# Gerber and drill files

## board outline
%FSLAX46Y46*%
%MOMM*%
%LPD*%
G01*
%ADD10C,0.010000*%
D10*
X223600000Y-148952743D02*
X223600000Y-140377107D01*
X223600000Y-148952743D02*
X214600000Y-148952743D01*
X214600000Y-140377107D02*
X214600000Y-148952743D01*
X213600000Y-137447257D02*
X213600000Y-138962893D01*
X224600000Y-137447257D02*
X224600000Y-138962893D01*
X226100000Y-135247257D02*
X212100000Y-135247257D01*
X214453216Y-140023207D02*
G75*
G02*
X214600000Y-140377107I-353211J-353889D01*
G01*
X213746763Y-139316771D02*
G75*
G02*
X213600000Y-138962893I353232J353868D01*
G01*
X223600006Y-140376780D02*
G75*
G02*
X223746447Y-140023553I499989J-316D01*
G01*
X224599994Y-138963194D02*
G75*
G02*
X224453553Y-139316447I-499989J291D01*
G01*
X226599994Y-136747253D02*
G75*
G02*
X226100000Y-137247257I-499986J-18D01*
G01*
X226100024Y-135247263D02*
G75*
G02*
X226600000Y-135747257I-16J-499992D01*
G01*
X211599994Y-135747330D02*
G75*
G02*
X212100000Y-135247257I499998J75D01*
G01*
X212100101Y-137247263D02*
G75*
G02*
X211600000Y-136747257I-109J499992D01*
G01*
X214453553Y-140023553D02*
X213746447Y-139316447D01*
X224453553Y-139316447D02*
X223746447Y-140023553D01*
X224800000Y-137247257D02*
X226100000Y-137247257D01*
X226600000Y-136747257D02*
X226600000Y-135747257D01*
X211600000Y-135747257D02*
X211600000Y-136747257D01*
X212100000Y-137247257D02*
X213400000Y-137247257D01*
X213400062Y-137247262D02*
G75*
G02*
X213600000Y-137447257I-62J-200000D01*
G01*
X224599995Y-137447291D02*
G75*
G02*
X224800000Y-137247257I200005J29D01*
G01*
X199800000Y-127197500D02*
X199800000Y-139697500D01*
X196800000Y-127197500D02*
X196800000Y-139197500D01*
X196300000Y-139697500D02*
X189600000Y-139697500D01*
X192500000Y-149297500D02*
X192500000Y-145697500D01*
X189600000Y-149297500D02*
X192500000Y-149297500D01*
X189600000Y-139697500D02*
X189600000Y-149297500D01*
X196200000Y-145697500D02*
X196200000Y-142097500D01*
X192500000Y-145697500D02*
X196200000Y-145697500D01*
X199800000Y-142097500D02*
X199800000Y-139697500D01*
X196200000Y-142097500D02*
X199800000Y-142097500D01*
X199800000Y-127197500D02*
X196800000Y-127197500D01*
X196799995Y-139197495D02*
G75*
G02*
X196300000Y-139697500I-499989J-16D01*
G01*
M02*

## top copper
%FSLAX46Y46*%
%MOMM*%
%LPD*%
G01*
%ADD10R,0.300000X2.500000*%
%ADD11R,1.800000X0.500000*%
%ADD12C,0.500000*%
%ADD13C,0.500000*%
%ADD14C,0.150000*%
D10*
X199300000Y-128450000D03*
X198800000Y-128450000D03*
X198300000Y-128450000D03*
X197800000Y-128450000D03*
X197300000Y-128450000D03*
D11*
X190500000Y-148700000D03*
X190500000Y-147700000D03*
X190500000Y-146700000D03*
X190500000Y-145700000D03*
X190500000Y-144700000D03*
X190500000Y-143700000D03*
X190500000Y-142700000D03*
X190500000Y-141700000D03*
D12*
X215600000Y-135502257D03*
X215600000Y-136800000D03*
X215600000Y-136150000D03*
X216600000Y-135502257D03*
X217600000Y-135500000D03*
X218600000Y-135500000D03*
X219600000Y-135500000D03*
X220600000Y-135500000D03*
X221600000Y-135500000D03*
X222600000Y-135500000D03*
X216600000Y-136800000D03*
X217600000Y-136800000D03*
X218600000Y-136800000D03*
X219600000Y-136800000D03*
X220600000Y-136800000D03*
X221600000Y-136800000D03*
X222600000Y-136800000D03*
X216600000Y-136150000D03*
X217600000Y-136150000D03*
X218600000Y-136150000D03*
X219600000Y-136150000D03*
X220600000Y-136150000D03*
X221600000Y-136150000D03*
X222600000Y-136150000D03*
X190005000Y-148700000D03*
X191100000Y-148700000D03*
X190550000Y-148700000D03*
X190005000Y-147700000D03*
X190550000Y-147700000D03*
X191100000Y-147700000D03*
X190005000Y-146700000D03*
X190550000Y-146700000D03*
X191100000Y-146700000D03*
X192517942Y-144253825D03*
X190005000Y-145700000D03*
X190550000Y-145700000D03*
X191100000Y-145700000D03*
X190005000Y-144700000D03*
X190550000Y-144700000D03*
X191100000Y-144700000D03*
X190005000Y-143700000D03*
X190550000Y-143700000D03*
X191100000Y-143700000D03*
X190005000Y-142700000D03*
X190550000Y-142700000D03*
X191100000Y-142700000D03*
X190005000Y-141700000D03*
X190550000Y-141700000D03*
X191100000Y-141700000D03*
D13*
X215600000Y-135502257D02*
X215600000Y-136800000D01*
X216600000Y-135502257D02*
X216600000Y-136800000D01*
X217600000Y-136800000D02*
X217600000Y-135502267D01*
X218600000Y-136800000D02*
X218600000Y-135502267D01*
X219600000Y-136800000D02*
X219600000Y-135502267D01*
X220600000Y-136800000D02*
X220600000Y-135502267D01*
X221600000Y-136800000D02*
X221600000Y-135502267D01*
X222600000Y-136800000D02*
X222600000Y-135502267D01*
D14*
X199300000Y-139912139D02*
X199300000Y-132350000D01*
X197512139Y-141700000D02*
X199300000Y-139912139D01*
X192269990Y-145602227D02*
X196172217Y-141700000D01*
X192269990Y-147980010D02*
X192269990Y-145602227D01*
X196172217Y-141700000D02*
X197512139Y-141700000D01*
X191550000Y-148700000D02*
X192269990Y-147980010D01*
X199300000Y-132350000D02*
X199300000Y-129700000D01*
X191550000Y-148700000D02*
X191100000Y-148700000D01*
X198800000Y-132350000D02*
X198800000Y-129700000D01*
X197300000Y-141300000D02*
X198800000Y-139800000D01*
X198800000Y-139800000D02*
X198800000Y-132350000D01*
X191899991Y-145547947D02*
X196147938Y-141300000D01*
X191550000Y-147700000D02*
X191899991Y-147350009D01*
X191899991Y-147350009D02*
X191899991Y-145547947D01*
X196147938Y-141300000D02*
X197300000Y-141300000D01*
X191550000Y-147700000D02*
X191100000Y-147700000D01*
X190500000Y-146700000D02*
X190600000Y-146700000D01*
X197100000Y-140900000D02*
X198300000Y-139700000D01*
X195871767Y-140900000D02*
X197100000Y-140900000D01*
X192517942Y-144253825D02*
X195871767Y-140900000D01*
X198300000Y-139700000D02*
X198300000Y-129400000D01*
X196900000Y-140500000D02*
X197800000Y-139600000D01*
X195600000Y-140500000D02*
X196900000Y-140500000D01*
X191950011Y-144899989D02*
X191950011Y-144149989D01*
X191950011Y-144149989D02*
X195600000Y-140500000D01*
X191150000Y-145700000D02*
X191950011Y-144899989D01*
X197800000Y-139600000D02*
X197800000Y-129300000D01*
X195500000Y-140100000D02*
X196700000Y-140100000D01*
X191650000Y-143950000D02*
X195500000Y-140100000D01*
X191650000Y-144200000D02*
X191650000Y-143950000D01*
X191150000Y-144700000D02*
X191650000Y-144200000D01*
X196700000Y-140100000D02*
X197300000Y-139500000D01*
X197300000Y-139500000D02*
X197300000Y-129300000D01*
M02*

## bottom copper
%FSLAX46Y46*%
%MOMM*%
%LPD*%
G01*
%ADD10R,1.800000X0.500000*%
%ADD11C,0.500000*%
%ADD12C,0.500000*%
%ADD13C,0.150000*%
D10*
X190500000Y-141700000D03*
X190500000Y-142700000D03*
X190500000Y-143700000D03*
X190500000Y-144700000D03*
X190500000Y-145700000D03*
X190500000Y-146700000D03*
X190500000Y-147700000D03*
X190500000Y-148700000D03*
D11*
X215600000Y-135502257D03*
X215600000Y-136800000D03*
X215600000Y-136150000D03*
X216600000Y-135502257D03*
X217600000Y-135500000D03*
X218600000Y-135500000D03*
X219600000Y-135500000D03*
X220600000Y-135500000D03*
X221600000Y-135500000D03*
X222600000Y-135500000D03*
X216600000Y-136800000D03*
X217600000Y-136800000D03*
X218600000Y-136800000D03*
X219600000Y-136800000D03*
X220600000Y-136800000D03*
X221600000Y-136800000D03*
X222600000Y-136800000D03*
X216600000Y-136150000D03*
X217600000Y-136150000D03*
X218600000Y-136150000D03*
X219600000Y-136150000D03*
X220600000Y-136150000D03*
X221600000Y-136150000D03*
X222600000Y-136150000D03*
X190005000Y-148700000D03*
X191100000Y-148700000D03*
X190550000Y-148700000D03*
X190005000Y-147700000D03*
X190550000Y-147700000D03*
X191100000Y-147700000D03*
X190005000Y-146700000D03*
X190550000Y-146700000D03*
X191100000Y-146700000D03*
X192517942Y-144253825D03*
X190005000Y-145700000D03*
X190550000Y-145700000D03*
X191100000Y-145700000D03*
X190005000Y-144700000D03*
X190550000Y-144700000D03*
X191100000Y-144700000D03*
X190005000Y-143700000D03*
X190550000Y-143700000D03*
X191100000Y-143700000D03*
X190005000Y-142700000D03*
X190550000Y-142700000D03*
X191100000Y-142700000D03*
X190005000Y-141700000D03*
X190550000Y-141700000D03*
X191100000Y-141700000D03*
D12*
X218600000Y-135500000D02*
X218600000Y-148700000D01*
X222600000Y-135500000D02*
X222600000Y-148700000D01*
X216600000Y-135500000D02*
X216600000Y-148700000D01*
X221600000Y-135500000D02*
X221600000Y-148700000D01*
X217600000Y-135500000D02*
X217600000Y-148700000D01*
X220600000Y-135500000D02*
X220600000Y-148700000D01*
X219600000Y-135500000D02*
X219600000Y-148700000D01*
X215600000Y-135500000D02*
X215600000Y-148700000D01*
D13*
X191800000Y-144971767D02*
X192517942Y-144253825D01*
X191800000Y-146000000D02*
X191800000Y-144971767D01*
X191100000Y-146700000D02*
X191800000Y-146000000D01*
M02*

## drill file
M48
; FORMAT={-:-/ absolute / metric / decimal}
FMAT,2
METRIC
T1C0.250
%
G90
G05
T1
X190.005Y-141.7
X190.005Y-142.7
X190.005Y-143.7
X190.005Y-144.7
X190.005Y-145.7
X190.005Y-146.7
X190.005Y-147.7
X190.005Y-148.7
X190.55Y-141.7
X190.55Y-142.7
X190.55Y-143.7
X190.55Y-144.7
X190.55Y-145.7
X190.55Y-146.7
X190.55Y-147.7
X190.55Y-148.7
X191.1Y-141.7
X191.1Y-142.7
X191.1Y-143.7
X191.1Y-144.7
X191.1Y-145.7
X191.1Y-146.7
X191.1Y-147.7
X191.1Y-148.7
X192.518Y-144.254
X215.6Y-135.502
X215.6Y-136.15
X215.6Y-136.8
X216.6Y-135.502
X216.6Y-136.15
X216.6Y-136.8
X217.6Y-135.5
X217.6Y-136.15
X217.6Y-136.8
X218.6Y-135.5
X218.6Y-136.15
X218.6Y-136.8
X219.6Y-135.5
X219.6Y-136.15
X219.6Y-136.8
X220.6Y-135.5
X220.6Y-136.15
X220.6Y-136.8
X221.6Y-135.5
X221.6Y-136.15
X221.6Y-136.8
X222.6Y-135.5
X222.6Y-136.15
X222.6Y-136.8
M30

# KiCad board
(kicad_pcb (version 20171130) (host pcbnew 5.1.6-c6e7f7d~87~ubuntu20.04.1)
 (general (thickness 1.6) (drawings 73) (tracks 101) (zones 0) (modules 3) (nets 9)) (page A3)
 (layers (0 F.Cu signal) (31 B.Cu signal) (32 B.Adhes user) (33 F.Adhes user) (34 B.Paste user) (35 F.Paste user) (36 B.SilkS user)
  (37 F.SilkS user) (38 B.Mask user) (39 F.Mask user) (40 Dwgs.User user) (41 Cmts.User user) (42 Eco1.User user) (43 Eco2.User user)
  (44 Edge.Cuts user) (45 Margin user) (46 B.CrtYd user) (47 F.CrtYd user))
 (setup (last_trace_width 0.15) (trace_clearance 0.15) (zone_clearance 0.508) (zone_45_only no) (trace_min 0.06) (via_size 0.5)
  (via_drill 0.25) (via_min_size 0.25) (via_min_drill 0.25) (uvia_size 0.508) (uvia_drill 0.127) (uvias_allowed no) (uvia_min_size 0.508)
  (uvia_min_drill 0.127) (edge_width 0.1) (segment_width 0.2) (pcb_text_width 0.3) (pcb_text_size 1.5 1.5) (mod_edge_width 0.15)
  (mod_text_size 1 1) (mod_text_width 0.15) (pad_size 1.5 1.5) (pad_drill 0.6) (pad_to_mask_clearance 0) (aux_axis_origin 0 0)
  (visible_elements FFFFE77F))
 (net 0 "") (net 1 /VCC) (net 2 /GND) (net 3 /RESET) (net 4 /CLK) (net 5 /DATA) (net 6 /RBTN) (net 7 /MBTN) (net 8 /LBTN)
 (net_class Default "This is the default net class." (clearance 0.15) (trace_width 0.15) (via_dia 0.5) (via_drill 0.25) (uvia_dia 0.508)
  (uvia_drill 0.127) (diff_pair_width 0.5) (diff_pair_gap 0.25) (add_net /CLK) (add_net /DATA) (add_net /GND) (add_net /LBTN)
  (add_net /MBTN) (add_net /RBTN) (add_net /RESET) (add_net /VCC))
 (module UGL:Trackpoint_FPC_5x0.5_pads (layer F.Cu) (at 198.3 128.45)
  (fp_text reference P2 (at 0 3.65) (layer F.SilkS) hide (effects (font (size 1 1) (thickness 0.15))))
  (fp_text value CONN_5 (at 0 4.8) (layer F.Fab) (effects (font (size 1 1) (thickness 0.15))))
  (pad 5 smd rect (at 1 0) (size 0.3 2.5) (layers F.Cu F.Paste F.Mask) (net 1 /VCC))
  (pad 4 smd rect (at 0.5 0) (size 0.3 2.5) (layers F.Cu F.Paste F.Mask) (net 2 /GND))
  (pad 3 smd rect (at 0 0) (size 0.3 2.5) (layers F.Cu F.Paste F.Mask) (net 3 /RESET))
  (pad 2 smd rect (at -0.5 0) (size 0.3 2.5) (layers F.Cu F.Paste F.Mask) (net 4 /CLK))
  (pad 1 smd rect (at -1 0) (size 0.3 2.5) (layers F.Cu F.Paste F.Mask) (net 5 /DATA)))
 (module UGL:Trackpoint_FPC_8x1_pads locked (layer F.Cu) (at 190.5 145.2 270)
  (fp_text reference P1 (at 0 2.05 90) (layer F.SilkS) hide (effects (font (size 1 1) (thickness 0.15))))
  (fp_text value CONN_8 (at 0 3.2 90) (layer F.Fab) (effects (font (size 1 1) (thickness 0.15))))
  (pad 8 smd rect (at 3.5 0 270) (size 0.5 1.8) (layers F.Cu F.Paste F.Mask) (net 1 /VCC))
  (pad 7 smd rect (at 2.5 0 270) (size 0.5 1.8) (layers F.Cu F.Paste F.Mask) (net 2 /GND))
  (pad 6 smd rect (at 1.5 0 270) (size 0.5 1.8) (layers F.Cu F.Paste F.Mask) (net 3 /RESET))
  (pad 5 smd rect (at 0.5 0 270) (size 0.5 1.8) (layers F.Cu F.Paste F.Mask) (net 4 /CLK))
  (pad 4 smd rect (at -0.5 0 270) (size 0.5 1.8) (layers F.Cu F.Paste F.Mask) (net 5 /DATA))
  (pad 3 smd rect (at -1.5 0 270) (size 0.5 1.8) (layers F.Cu F.Paste F.Mask) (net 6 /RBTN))
  (pad 2 smd rect (at -2.5 0 270) (size 0.5 1.8) (layers F.Cu F.Paste F.Mask) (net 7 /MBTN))
  (pad 1 smd rect (at -3.5 0 270) (size 0.5 1.8) (layers F.Cu F.Paste F.Mask) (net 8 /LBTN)))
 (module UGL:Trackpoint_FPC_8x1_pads (layer B.Cu) (at 190.5 145.2 270)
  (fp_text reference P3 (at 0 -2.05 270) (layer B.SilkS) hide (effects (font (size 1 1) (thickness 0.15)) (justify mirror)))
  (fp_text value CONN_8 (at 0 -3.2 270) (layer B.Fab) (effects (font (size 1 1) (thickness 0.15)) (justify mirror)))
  (pad 1 smd rect (at -3.5 0 270) (size 0.5 1.8) (layers B.Cu B.Paste B.Mask) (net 8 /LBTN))
  (pad 2 smd rect (at -2.5 0 270) (size 0.5 1.8) (layers B.Cu B.Paste B.Mask) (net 7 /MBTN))
  (pad 3 smd rect (at -1.5 0 270) (size 0.5 1.8) (layers B.Cu B.Paste B.Mask) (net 6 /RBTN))
  (pad 4 smd rect (at -0.5 0 270) (size 0.5 1.8) (layers B.Cu B.Paste B.Mask) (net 5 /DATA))
  (pad 5 smd rect (at 0.5 0 270) (size 0.5 1.8) (layers B.Cu B.Paste B.Mask) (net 4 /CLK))
  (pad 6 smd rect (at 1.5 0 270) (size 0.5 1.8) (layers B.Cu B.Paste B.Mask) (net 3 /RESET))
  (pad 7 smd rect (at 2.5 0 270) (size 0.5 1.8) (layers B.Cu B.Paste B.Mask) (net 2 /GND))
  (pad 8 smd rect (at 3.5 0 270) (size 0.5 1.8) (layers B.Cu B.Paste B.Mask) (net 1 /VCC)))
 (gr_line (start 223.6 148.952743) (end 223.6 140.377107) (angle 90) (layer Edge.Cuts) (width 0.01))
 (gr_line (start 223.6 148.952743) (end 214.6 148.952743) (angle 90) (layer Edge.Cuts) (width 0.01))
 (gr_line (start 214.6 140.377107) (end 214.6 148.952743) (angle 90) (layer Edge.Cuts) (width 0.01))
 (gr_line (start 213.6 137.447257) (end 213.6 138.962893) (angle 90) (layer Edge.Cuts) (width 0.01))
 (gr_line (start 224.6 137.447257) (end 224.6 138.962893) (angle 90) (layer Edge.Cuts) (width 0.01))
 (gr_line (start 226.1 135.247257) (end 212.1 135.247257) (angle 90) (layer Edge.Cuts) (width 0.01))
 (gr_arc (start 214.100005 140.377096) (end 214.6 140.377107) (angle -45.0562246) (layer Edge.Cuts) (width 0.01))
 (gr_arc (start 214.099995 138.962903) (end 213.6 138.962893) (angle -45.05269373) (layer Edge.Cuts) (width 0.01))
 (gr_arc (start 224.099995 140.377096) (end 223.746447 140.023553) (angle -44.96338237) (layer Edge.Cuts) (width 0.01))
 (gr_arc (start 224.100005 138.962903) (end 224.453553 139.316447) (angle -44.96638194) (layer Edge.Cuts) (width 0.01))
 (gr_arc (start 226.100008 136.747271) (end 226.1 137.247257) (angle -90.00303091) (layer Edge.Cuts) (width 0.01))
 (gr_arc (start 226.100008 135.747255) (end 226.6 135.747257) (angle -89.99845171) (layer Edge.Cuts) (width 0.01))
 (gr_arc (start 212.099992 135.747255) (end 212.1 135.247257) (angle -90.00950545) (layer Edge.Cuts) (width 0.01))
 (gr_arc (start 212.099992 136.747271) (end 211.6 136.747257) (angle -90.01408384) (layer Edge.Cuts) (width 0.01))
 (gr_line (start 214.453553 140.023553) (end 213.746447 139.316447) (angle 90) (layer Edge.Cuts) (width 0.01))
 (gr_line (start 224.453553 139.316447) (end 223.746447 140.023553) (angle 90) (layer Edge.Cuts) (width 0.01))
 (gr_line (start 224.8 137.247257) (end 226.1 137.247257) (angle 90) (layer Edge.Cuts) (width 0.01))
 (gr_line (start 226.6 136.747257) (end 226.6 135.747257) (angle 90) (layer Edge.Cuts) (width 0.01))
 (gr_line (start 211.6 135.747257) (end 211.6 136.747257) (angle 90) (layer Edge.Cuts) (width 0.01))
 (gr_line (start 212.1 137.247257) (end 213.4 137.247257) (angle 90) (layer Edge.Cuts) (width 0.01))
 (gr_arc (start 213.4 137.447262) (end 213.6 137.447257) (angle -89.98075418) (layer Edge.Cuts) (width 0.01))
 (gr_arc (start 224.8 137.447262) (end 224.8 137.247257) (angle -90.00839267) (layer Edge.Cuts) (width 0.01))
 (gr_line (start 199.8 127.1975) (end 199.8 139.6975) (angle 90) (layer Edge.Cuts) (width 0.01))
 (gr_line (start 196.8 127.1975) (end 196.8 139.1975) (angle 90) (layer Edge.Cuts) (width 0.01))
 (gr_line (start 196.3 139.6975) (end 189.6 139.6975) (angle 90) (layer Edge.Cuts) (width 0.01))
 (gr_line (start 192.5 149.2975) (end 192.5 145.6975) (angle 90) (layer Edge.Cuts) (width 0.01))
 (gr_line (start 189.6 149.2975) (end 192.5 149.2975) (angle 90) (layer Edge.Cuts) (width 0.01))
 (gr_line (start 189.6 139.6975) (end 189.6 149.2975) (angle 90) (layer Edge.Cuts) (width 0.01))
 (gr_line (start 196.2 145.6975) (end 196.2 142.0975) (angle 90) (layer Edge.Cuts) (width 0.01))
 (gr_line (start 192.5 145.6975) (end 196.2 145.6975) (angle 90) (layer Edge.Cuts) (width 0.01))
 (gr_line (start 199.8 142.0975) (end 199.8 139.6975) (angle 90) (layer Edge.Cuts) (width 0.01))
 (gr_line (start 196.2 142.0975) (end 199.8 142.0975) (angle 90) (layer Edge.Cuts) (width 0.01))
 (gr_line (start 199.8 127.1975) (end 196.8 127.1975) (angle 90) (layer Edge.Cuts) (width 0.01))
 (gr_arc (start 196.300006 139.197511) (end 196.3 139.6975) (angle -90.00254177) (layer Edge.Cuts) (width 0.01))
 (via (at 215.6 135.502257) (size 0.5) (drill 0.25) (layers F.Cu B.Cu) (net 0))
 (via (at 215.6 136.8) (size 0.5) (drill 0.25) (layers F.Cu B.Cu) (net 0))
 (via (at 215.6 136.15) (size 0.5) (drill 0.25) (layers F.Cu B.Cu) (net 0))
 (via (at 216.6 135.502257) (size 0.5) (drill 0.25) (layers F.Cu B.Cu) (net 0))
 (via (at 217.6 135.5) (size 0.5) (drill 0.25) (layers F.Cu B.Cu) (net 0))
 (via (at 218.6 135.5) (size 0.5) (drill 0.25) (layers F.Cu B.Cu) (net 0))
 (via (at 219.6 135.5) (size 0.5) (drill 0.25) (layers F.Cu B.Cu) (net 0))
 (via (at 220.6 135.5) (size 0.5) (drill 0.25) (layers F.Cu B.Cu) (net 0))
 (via (at 221.6 135.5) (size 0.5) (drill 0.25) (layers F.Cu B.Cu) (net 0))
 (via (at 222.6 135.5) (size 0.5) (drill 0.25) (layers F.Cu B.Cu) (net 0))
 (via (at 216.6 136.8) (size 0.5) (drill 0.25) (layers F.Cu B.Cu) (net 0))
 (via (at 217.6 136.8) (size 0.5) (drill 0.25) (layers F.Cu B.Cu) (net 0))
 (via (at 218.6 136.8) (size 0.5) (drill 0.25) (layers F.Cu B.Cu) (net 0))
 (via (at 219.6 136.8) (size 0.5) (drill 0.25) (layers F.Cu B.Cu) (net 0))
 (via (at 220.6 136.8) (size 0.5) (drill 0.25) (layers F.Cu B.Cu) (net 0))
 (via (at 221.6 136.8) (size 0.5) (drill 0.25) (layers F.Cu B.Cu) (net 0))
 (via (at 222.6 136.8) (size 0.5) (drill 0.25) (layers F.Cu B.Cu) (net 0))
 (via (at 216.6 136.15) (size 0.5) (drill 0.25) (layers F.Cu B.Cu) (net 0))
 (via (at 217.6 136.15) (size 0.5) (drill 0.25) (layers F.Cu B.Cu) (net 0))
 (via (at 218.6 136.15) (size 0.5) (drill 0.25) (layers F.Cu B.Cu) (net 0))
 (via (at 219.6 136.15) (size 0.5) (drill 0.25) (layers F.Cu B.Cu) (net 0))
 (via (at 220.6 136.15) (size 0.5) (drill 0.25) (layers F.Cu B.Cu) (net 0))
 (via (at 221.6 136.15) (size 0.5) (drill 0.25) (layers F.Cu B.Cu) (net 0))
 (via (at 222.6 136.15) (size 0.5) (drill 0.25) (layers F.Cu B.Cu) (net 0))
 (segment (start 215.6 135.502257) (end 215.6 136.8) (width 0.5) (layer F.Cu) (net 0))
 (segment (start 216.6 135.502257) (end 216.6 136.8) (width 0.5) (layer F.Cu) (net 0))
 (segment (start 217.6 136.8) (end 217.6 135.502267) (width 0.5) (layer F.Cu) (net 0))
 (segment (start 218.6 136.8) (end 218.6 135.502267) (width 0.5) (layer F.Cu) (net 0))
 (segment (start 219.6 136.8) (end 219.6 135.502267) (width 0.5) (layer F.Cu) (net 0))
 (segment (start 220.6 136.8) (end 220.6 135.502267) (width 0.5) (layer F.Cu) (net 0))
 (segment (start 221.6 136.8) (end 221.6 135.502267) (width 0.5) (layer F.Cu) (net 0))
 (segment (start 222.6 136.8) (end 222.6 135.502267) (width 0.5) (layer F.Cu) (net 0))
 (segment (start 218.6 135.5) (end 218.6 148.7) (width 0.5) (layer B.Cu) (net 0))
 (segment (start 222.6 135.5) (end 222.6 148.7) (width 0.5) (layer B.Cu) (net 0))
 (segment (start 216.6 135.5) (end 216.6 148.7) (width 0.5) (layer B.Cu) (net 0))
 (segment (start 221.6 135.5) (end 221.6 148.7) (width 0.5) (layer B.Cu) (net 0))
 (segment (start 217.6 135.5) (end 217.6 148.7) (width 0.5) (layer B.Cu) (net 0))
 (segment (start 220.6 135.5) (end 220.6 148.7) (width 0.5) (layer B.Cu) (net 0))
 (segment (start 219.6 135.5) (end 219.6 148.7) (width 0.5) (layer B.Cu) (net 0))
 (segment (start 215.6 135.5) (end 215.6 148.7) (width 0.5) (layer B.Cu) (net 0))
 (segment (start 199.3 139.912139) (end 199.3 132.35) (width 0.15) (layer F.Cu) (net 1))
 (segment (start 197.512139 141.7) (end 199.3 139.912139) (width 0.15) (layer F.Cu) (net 1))
 (segment (start 192.26999 145.602227) (end 196.172217 141.7) (width 0.15) (layer F.Cu) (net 1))
 (segment (start 192.26999 147.98001) (end 192.26999 145.602227) (width 0.15) (layer F.Cu) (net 1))
 (segment (start 196.172217 141.7) (end 197.512139 141.7) (width 0.15) (layer F.Cu) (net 1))
 (segment (start 191.55 148.7) (end 192.26999 147.98001) (width 0.15) (layer F.Cu) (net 1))
 (segment (start 199.3 132.35) (end 199.3 129.7) (width 0.15) (layer F.Cu) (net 1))
 (via (at 190.005 148.7) (size 0.5) (drill 0.25) (layers F.Cu B.Cu) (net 1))
 (via (at 191.1 148.7) (size 0.5) (drill 0.25) (layers F.Cu B.Cu) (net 1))
 (via (at 190.55 148.7) (size 0.5) (drill 0.25) (layers F.Cu B.Cu) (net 1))
 (segment (start 191.55 148.7) (end 191.1 148.7) (width 0.15) (layer F.Cu) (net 1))
 (segment (start 198.8 132.35) (end 198.8 129.7) (width 0.15) (layer F.Cu) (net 2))
 (segment (start 197.3 141.3) (end 198.8 139.8) (width 0.15) (layer F.Cu) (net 2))
 (segment (start 198.8 139.8) (end 198.8 132.35) (width 0.15) (layer F.Cu) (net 2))
 (segment (start 191.899991 145.547947) (end 196.147938 141.3) (width 0.15) (layer F.Cu) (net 2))
 (segment (start 191.55 147.7) (end 191.899991 147.350009) (width 0.15) (layer F.Cu) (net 2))
 (segment (start 191.899991 147.350009) (end 191.899991 145.547947) (width 0.15) (layer F.Cu) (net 2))
 (segment (start 196.147938 141.3) (end 197.3 141.3) (width 0.15) (layer F.Cu) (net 2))
 (via (at 190.005 147.7) (size 0.5) (drill 0.25) (layers F.Cu B.Cu) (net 2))
 (via (at 190.55 147.7) (size 0.5) (drill 0.25) (layers F.Cu B.Cu) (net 2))
 (via (at 191.1 147.7) (size 0.5) (drill 0.25) (layers F.Cu B.Cu) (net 2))
 (segment (start 191.55 147.7) (end 191.1 147.7) (width 0.15) (layer F.Cu) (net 2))
 (via (at 190.005 146.7) (size 0.5) (drill 0.25) (layers F.Cu B.Cu) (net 3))
 (via (at 190.55 146.7) (size 0.5) (drill 0.25) (layers F.Cu B.Cu) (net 3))
 (segment (start 190.5 146.7) (end 190.6 146.7) (width 0.15) (layer F.Cu) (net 3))
 (via (at 191.1 146.7) (size 0.5) (drill 0.25) (layers F.Cu B.Cu) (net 3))
 (via (at 192.517942 144.253825) (size 0.5) (drill 0.25) (layers F.Cu B.Cu) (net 3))
 (segment (start 197.1 140.9) (end 198.3 139.7) (width 0.15) (layer F.Cu) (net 3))
 (segment (start 195.871767 140.9) (end 197.1 140.9) (width 0.15) (layer F.Cu) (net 3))
 (segment (start 192.517942 144.253825) (end 195.871767 140.9) (width 0.15) (layer F.Cu) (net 3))
 (segment (start 191.8 144.971767) (end 192.517942 144.253825) (width 0.15) (layer B.Cu) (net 3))
 (segment (start 191.8 146) (end 191.8 144.971767) (width 0.15) (layer B.Cu) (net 3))
 (segment (start 191.1 146.7) (end 191.8 146) (width 0.15) (layer B.Cu) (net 3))
 (segment (start 198.3 139.7) (end 198.3 129.4) (width 0.15) (layer F.Cu) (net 3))
 (segment (start 196.9 140.5) (end 197.8 139.6) (width 0.15) (layer F.Cu) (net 4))
 (segment (start 195.6 140.5) (end 196.9 140.5) (width 0.15) (layer F.Cu) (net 4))
 (segment (start 191.950011 144.899989) (end 191.950011 144.149989) (width 0.15) (layer F.Cu) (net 4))
 (segment (start 191.950011 144.149989) (end 195.6 140.5) (width 0.15) (layer F.Cu) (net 4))
 (segment (start 191.15 145.7) (end 191.950011 144.899989) (width 0.15) (layer F.Cu) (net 4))
 (via (at 190.005 145.7) (size 0.5) (drill 0.25) (layers F.Cu B.Cu) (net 4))
 (via (at 190.55 145.7) (size 0.5) (drill 0.25) (layers F.Cu B.Cu) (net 4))
 (via (at 191.1 145.7) (size 0.5) (drill 0.25) (layers F.Cu B.Cu) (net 4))
 (segment (start 197.8 139.6) (end 197.8 129.3) (width 0.15) (layer F.Cu) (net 4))
 (segment (start 195.5 140.1) (end 196.7 140.1) (width 0.15) (layer F.Cu) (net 5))
 (segment (start 191.65 143.95) (end 195.5 140.1) (width 0.15) (layer F.Cu) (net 5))
 (segment (start 191.65 144.2) (end 191.65 143.95) (width 0.15) (layer F.Cu) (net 5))
 (segment (start 191.15 144.7) (end 191.65 144.2) (width 0.15) (layer F.Cu) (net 5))
 (segment (start 196.7 140.1) (end 197.3 139.5) (width 0.15) (layer F.Cu) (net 5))
 (via (at 190.005 144.7) (size 0.5) (drill 0.25) (layers F.Cu B.Cu) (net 5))
 (via (at 190.55 144.7) (size 0.5) (drill 0.25) (layers F.Cu B.Cu) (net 5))
 (via (at 191.1 144.7) (size 0.5) (drill 0.25) (layers F.Cu B.Cu) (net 5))
 (segment (start 197.3 139.5) (end 197.3 129.3) (width 0.15) (layer F.Cu) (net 5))
 (via (at 190.005 143.7) (size 0.5) (drill 0.25) (layers F.Cu B.Cu) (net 6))
 (via (at 190.55 143.7) (size 0.5) (drill 0.25) (layers F.Cu B.Cu) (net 6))
 (via (at 191.1 143.7) (size 0.5) (drill 0.25) (layers F.Cu B.Cu) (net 6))
 (via (at 190.005 142.7) (size 0.5) (drill 0.25) (layers F.Cu B.Cu) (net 7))
 (via (at 190.55 142.7) (size 0.5) (drill 0.25) (layers F.Cu B.Cu) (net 7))
 (via (at 191.1 142.7) (size 0.5) (drill 0.25) (layers F.Cu B.Cu) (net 7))
 (via (at 190.005 141.7) (size 0.5) (drill 0.25) (layers F.Cu B.Cu) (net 8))
 (via (at 190.55 141.7) (size 0.5) (drill 0.25) (layers F.Cu B.Cu) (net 8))
 (via (at 191.1 141.7) (size 0.5) (drill 0.25) (layers F.Cu B.Cu) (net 8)))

